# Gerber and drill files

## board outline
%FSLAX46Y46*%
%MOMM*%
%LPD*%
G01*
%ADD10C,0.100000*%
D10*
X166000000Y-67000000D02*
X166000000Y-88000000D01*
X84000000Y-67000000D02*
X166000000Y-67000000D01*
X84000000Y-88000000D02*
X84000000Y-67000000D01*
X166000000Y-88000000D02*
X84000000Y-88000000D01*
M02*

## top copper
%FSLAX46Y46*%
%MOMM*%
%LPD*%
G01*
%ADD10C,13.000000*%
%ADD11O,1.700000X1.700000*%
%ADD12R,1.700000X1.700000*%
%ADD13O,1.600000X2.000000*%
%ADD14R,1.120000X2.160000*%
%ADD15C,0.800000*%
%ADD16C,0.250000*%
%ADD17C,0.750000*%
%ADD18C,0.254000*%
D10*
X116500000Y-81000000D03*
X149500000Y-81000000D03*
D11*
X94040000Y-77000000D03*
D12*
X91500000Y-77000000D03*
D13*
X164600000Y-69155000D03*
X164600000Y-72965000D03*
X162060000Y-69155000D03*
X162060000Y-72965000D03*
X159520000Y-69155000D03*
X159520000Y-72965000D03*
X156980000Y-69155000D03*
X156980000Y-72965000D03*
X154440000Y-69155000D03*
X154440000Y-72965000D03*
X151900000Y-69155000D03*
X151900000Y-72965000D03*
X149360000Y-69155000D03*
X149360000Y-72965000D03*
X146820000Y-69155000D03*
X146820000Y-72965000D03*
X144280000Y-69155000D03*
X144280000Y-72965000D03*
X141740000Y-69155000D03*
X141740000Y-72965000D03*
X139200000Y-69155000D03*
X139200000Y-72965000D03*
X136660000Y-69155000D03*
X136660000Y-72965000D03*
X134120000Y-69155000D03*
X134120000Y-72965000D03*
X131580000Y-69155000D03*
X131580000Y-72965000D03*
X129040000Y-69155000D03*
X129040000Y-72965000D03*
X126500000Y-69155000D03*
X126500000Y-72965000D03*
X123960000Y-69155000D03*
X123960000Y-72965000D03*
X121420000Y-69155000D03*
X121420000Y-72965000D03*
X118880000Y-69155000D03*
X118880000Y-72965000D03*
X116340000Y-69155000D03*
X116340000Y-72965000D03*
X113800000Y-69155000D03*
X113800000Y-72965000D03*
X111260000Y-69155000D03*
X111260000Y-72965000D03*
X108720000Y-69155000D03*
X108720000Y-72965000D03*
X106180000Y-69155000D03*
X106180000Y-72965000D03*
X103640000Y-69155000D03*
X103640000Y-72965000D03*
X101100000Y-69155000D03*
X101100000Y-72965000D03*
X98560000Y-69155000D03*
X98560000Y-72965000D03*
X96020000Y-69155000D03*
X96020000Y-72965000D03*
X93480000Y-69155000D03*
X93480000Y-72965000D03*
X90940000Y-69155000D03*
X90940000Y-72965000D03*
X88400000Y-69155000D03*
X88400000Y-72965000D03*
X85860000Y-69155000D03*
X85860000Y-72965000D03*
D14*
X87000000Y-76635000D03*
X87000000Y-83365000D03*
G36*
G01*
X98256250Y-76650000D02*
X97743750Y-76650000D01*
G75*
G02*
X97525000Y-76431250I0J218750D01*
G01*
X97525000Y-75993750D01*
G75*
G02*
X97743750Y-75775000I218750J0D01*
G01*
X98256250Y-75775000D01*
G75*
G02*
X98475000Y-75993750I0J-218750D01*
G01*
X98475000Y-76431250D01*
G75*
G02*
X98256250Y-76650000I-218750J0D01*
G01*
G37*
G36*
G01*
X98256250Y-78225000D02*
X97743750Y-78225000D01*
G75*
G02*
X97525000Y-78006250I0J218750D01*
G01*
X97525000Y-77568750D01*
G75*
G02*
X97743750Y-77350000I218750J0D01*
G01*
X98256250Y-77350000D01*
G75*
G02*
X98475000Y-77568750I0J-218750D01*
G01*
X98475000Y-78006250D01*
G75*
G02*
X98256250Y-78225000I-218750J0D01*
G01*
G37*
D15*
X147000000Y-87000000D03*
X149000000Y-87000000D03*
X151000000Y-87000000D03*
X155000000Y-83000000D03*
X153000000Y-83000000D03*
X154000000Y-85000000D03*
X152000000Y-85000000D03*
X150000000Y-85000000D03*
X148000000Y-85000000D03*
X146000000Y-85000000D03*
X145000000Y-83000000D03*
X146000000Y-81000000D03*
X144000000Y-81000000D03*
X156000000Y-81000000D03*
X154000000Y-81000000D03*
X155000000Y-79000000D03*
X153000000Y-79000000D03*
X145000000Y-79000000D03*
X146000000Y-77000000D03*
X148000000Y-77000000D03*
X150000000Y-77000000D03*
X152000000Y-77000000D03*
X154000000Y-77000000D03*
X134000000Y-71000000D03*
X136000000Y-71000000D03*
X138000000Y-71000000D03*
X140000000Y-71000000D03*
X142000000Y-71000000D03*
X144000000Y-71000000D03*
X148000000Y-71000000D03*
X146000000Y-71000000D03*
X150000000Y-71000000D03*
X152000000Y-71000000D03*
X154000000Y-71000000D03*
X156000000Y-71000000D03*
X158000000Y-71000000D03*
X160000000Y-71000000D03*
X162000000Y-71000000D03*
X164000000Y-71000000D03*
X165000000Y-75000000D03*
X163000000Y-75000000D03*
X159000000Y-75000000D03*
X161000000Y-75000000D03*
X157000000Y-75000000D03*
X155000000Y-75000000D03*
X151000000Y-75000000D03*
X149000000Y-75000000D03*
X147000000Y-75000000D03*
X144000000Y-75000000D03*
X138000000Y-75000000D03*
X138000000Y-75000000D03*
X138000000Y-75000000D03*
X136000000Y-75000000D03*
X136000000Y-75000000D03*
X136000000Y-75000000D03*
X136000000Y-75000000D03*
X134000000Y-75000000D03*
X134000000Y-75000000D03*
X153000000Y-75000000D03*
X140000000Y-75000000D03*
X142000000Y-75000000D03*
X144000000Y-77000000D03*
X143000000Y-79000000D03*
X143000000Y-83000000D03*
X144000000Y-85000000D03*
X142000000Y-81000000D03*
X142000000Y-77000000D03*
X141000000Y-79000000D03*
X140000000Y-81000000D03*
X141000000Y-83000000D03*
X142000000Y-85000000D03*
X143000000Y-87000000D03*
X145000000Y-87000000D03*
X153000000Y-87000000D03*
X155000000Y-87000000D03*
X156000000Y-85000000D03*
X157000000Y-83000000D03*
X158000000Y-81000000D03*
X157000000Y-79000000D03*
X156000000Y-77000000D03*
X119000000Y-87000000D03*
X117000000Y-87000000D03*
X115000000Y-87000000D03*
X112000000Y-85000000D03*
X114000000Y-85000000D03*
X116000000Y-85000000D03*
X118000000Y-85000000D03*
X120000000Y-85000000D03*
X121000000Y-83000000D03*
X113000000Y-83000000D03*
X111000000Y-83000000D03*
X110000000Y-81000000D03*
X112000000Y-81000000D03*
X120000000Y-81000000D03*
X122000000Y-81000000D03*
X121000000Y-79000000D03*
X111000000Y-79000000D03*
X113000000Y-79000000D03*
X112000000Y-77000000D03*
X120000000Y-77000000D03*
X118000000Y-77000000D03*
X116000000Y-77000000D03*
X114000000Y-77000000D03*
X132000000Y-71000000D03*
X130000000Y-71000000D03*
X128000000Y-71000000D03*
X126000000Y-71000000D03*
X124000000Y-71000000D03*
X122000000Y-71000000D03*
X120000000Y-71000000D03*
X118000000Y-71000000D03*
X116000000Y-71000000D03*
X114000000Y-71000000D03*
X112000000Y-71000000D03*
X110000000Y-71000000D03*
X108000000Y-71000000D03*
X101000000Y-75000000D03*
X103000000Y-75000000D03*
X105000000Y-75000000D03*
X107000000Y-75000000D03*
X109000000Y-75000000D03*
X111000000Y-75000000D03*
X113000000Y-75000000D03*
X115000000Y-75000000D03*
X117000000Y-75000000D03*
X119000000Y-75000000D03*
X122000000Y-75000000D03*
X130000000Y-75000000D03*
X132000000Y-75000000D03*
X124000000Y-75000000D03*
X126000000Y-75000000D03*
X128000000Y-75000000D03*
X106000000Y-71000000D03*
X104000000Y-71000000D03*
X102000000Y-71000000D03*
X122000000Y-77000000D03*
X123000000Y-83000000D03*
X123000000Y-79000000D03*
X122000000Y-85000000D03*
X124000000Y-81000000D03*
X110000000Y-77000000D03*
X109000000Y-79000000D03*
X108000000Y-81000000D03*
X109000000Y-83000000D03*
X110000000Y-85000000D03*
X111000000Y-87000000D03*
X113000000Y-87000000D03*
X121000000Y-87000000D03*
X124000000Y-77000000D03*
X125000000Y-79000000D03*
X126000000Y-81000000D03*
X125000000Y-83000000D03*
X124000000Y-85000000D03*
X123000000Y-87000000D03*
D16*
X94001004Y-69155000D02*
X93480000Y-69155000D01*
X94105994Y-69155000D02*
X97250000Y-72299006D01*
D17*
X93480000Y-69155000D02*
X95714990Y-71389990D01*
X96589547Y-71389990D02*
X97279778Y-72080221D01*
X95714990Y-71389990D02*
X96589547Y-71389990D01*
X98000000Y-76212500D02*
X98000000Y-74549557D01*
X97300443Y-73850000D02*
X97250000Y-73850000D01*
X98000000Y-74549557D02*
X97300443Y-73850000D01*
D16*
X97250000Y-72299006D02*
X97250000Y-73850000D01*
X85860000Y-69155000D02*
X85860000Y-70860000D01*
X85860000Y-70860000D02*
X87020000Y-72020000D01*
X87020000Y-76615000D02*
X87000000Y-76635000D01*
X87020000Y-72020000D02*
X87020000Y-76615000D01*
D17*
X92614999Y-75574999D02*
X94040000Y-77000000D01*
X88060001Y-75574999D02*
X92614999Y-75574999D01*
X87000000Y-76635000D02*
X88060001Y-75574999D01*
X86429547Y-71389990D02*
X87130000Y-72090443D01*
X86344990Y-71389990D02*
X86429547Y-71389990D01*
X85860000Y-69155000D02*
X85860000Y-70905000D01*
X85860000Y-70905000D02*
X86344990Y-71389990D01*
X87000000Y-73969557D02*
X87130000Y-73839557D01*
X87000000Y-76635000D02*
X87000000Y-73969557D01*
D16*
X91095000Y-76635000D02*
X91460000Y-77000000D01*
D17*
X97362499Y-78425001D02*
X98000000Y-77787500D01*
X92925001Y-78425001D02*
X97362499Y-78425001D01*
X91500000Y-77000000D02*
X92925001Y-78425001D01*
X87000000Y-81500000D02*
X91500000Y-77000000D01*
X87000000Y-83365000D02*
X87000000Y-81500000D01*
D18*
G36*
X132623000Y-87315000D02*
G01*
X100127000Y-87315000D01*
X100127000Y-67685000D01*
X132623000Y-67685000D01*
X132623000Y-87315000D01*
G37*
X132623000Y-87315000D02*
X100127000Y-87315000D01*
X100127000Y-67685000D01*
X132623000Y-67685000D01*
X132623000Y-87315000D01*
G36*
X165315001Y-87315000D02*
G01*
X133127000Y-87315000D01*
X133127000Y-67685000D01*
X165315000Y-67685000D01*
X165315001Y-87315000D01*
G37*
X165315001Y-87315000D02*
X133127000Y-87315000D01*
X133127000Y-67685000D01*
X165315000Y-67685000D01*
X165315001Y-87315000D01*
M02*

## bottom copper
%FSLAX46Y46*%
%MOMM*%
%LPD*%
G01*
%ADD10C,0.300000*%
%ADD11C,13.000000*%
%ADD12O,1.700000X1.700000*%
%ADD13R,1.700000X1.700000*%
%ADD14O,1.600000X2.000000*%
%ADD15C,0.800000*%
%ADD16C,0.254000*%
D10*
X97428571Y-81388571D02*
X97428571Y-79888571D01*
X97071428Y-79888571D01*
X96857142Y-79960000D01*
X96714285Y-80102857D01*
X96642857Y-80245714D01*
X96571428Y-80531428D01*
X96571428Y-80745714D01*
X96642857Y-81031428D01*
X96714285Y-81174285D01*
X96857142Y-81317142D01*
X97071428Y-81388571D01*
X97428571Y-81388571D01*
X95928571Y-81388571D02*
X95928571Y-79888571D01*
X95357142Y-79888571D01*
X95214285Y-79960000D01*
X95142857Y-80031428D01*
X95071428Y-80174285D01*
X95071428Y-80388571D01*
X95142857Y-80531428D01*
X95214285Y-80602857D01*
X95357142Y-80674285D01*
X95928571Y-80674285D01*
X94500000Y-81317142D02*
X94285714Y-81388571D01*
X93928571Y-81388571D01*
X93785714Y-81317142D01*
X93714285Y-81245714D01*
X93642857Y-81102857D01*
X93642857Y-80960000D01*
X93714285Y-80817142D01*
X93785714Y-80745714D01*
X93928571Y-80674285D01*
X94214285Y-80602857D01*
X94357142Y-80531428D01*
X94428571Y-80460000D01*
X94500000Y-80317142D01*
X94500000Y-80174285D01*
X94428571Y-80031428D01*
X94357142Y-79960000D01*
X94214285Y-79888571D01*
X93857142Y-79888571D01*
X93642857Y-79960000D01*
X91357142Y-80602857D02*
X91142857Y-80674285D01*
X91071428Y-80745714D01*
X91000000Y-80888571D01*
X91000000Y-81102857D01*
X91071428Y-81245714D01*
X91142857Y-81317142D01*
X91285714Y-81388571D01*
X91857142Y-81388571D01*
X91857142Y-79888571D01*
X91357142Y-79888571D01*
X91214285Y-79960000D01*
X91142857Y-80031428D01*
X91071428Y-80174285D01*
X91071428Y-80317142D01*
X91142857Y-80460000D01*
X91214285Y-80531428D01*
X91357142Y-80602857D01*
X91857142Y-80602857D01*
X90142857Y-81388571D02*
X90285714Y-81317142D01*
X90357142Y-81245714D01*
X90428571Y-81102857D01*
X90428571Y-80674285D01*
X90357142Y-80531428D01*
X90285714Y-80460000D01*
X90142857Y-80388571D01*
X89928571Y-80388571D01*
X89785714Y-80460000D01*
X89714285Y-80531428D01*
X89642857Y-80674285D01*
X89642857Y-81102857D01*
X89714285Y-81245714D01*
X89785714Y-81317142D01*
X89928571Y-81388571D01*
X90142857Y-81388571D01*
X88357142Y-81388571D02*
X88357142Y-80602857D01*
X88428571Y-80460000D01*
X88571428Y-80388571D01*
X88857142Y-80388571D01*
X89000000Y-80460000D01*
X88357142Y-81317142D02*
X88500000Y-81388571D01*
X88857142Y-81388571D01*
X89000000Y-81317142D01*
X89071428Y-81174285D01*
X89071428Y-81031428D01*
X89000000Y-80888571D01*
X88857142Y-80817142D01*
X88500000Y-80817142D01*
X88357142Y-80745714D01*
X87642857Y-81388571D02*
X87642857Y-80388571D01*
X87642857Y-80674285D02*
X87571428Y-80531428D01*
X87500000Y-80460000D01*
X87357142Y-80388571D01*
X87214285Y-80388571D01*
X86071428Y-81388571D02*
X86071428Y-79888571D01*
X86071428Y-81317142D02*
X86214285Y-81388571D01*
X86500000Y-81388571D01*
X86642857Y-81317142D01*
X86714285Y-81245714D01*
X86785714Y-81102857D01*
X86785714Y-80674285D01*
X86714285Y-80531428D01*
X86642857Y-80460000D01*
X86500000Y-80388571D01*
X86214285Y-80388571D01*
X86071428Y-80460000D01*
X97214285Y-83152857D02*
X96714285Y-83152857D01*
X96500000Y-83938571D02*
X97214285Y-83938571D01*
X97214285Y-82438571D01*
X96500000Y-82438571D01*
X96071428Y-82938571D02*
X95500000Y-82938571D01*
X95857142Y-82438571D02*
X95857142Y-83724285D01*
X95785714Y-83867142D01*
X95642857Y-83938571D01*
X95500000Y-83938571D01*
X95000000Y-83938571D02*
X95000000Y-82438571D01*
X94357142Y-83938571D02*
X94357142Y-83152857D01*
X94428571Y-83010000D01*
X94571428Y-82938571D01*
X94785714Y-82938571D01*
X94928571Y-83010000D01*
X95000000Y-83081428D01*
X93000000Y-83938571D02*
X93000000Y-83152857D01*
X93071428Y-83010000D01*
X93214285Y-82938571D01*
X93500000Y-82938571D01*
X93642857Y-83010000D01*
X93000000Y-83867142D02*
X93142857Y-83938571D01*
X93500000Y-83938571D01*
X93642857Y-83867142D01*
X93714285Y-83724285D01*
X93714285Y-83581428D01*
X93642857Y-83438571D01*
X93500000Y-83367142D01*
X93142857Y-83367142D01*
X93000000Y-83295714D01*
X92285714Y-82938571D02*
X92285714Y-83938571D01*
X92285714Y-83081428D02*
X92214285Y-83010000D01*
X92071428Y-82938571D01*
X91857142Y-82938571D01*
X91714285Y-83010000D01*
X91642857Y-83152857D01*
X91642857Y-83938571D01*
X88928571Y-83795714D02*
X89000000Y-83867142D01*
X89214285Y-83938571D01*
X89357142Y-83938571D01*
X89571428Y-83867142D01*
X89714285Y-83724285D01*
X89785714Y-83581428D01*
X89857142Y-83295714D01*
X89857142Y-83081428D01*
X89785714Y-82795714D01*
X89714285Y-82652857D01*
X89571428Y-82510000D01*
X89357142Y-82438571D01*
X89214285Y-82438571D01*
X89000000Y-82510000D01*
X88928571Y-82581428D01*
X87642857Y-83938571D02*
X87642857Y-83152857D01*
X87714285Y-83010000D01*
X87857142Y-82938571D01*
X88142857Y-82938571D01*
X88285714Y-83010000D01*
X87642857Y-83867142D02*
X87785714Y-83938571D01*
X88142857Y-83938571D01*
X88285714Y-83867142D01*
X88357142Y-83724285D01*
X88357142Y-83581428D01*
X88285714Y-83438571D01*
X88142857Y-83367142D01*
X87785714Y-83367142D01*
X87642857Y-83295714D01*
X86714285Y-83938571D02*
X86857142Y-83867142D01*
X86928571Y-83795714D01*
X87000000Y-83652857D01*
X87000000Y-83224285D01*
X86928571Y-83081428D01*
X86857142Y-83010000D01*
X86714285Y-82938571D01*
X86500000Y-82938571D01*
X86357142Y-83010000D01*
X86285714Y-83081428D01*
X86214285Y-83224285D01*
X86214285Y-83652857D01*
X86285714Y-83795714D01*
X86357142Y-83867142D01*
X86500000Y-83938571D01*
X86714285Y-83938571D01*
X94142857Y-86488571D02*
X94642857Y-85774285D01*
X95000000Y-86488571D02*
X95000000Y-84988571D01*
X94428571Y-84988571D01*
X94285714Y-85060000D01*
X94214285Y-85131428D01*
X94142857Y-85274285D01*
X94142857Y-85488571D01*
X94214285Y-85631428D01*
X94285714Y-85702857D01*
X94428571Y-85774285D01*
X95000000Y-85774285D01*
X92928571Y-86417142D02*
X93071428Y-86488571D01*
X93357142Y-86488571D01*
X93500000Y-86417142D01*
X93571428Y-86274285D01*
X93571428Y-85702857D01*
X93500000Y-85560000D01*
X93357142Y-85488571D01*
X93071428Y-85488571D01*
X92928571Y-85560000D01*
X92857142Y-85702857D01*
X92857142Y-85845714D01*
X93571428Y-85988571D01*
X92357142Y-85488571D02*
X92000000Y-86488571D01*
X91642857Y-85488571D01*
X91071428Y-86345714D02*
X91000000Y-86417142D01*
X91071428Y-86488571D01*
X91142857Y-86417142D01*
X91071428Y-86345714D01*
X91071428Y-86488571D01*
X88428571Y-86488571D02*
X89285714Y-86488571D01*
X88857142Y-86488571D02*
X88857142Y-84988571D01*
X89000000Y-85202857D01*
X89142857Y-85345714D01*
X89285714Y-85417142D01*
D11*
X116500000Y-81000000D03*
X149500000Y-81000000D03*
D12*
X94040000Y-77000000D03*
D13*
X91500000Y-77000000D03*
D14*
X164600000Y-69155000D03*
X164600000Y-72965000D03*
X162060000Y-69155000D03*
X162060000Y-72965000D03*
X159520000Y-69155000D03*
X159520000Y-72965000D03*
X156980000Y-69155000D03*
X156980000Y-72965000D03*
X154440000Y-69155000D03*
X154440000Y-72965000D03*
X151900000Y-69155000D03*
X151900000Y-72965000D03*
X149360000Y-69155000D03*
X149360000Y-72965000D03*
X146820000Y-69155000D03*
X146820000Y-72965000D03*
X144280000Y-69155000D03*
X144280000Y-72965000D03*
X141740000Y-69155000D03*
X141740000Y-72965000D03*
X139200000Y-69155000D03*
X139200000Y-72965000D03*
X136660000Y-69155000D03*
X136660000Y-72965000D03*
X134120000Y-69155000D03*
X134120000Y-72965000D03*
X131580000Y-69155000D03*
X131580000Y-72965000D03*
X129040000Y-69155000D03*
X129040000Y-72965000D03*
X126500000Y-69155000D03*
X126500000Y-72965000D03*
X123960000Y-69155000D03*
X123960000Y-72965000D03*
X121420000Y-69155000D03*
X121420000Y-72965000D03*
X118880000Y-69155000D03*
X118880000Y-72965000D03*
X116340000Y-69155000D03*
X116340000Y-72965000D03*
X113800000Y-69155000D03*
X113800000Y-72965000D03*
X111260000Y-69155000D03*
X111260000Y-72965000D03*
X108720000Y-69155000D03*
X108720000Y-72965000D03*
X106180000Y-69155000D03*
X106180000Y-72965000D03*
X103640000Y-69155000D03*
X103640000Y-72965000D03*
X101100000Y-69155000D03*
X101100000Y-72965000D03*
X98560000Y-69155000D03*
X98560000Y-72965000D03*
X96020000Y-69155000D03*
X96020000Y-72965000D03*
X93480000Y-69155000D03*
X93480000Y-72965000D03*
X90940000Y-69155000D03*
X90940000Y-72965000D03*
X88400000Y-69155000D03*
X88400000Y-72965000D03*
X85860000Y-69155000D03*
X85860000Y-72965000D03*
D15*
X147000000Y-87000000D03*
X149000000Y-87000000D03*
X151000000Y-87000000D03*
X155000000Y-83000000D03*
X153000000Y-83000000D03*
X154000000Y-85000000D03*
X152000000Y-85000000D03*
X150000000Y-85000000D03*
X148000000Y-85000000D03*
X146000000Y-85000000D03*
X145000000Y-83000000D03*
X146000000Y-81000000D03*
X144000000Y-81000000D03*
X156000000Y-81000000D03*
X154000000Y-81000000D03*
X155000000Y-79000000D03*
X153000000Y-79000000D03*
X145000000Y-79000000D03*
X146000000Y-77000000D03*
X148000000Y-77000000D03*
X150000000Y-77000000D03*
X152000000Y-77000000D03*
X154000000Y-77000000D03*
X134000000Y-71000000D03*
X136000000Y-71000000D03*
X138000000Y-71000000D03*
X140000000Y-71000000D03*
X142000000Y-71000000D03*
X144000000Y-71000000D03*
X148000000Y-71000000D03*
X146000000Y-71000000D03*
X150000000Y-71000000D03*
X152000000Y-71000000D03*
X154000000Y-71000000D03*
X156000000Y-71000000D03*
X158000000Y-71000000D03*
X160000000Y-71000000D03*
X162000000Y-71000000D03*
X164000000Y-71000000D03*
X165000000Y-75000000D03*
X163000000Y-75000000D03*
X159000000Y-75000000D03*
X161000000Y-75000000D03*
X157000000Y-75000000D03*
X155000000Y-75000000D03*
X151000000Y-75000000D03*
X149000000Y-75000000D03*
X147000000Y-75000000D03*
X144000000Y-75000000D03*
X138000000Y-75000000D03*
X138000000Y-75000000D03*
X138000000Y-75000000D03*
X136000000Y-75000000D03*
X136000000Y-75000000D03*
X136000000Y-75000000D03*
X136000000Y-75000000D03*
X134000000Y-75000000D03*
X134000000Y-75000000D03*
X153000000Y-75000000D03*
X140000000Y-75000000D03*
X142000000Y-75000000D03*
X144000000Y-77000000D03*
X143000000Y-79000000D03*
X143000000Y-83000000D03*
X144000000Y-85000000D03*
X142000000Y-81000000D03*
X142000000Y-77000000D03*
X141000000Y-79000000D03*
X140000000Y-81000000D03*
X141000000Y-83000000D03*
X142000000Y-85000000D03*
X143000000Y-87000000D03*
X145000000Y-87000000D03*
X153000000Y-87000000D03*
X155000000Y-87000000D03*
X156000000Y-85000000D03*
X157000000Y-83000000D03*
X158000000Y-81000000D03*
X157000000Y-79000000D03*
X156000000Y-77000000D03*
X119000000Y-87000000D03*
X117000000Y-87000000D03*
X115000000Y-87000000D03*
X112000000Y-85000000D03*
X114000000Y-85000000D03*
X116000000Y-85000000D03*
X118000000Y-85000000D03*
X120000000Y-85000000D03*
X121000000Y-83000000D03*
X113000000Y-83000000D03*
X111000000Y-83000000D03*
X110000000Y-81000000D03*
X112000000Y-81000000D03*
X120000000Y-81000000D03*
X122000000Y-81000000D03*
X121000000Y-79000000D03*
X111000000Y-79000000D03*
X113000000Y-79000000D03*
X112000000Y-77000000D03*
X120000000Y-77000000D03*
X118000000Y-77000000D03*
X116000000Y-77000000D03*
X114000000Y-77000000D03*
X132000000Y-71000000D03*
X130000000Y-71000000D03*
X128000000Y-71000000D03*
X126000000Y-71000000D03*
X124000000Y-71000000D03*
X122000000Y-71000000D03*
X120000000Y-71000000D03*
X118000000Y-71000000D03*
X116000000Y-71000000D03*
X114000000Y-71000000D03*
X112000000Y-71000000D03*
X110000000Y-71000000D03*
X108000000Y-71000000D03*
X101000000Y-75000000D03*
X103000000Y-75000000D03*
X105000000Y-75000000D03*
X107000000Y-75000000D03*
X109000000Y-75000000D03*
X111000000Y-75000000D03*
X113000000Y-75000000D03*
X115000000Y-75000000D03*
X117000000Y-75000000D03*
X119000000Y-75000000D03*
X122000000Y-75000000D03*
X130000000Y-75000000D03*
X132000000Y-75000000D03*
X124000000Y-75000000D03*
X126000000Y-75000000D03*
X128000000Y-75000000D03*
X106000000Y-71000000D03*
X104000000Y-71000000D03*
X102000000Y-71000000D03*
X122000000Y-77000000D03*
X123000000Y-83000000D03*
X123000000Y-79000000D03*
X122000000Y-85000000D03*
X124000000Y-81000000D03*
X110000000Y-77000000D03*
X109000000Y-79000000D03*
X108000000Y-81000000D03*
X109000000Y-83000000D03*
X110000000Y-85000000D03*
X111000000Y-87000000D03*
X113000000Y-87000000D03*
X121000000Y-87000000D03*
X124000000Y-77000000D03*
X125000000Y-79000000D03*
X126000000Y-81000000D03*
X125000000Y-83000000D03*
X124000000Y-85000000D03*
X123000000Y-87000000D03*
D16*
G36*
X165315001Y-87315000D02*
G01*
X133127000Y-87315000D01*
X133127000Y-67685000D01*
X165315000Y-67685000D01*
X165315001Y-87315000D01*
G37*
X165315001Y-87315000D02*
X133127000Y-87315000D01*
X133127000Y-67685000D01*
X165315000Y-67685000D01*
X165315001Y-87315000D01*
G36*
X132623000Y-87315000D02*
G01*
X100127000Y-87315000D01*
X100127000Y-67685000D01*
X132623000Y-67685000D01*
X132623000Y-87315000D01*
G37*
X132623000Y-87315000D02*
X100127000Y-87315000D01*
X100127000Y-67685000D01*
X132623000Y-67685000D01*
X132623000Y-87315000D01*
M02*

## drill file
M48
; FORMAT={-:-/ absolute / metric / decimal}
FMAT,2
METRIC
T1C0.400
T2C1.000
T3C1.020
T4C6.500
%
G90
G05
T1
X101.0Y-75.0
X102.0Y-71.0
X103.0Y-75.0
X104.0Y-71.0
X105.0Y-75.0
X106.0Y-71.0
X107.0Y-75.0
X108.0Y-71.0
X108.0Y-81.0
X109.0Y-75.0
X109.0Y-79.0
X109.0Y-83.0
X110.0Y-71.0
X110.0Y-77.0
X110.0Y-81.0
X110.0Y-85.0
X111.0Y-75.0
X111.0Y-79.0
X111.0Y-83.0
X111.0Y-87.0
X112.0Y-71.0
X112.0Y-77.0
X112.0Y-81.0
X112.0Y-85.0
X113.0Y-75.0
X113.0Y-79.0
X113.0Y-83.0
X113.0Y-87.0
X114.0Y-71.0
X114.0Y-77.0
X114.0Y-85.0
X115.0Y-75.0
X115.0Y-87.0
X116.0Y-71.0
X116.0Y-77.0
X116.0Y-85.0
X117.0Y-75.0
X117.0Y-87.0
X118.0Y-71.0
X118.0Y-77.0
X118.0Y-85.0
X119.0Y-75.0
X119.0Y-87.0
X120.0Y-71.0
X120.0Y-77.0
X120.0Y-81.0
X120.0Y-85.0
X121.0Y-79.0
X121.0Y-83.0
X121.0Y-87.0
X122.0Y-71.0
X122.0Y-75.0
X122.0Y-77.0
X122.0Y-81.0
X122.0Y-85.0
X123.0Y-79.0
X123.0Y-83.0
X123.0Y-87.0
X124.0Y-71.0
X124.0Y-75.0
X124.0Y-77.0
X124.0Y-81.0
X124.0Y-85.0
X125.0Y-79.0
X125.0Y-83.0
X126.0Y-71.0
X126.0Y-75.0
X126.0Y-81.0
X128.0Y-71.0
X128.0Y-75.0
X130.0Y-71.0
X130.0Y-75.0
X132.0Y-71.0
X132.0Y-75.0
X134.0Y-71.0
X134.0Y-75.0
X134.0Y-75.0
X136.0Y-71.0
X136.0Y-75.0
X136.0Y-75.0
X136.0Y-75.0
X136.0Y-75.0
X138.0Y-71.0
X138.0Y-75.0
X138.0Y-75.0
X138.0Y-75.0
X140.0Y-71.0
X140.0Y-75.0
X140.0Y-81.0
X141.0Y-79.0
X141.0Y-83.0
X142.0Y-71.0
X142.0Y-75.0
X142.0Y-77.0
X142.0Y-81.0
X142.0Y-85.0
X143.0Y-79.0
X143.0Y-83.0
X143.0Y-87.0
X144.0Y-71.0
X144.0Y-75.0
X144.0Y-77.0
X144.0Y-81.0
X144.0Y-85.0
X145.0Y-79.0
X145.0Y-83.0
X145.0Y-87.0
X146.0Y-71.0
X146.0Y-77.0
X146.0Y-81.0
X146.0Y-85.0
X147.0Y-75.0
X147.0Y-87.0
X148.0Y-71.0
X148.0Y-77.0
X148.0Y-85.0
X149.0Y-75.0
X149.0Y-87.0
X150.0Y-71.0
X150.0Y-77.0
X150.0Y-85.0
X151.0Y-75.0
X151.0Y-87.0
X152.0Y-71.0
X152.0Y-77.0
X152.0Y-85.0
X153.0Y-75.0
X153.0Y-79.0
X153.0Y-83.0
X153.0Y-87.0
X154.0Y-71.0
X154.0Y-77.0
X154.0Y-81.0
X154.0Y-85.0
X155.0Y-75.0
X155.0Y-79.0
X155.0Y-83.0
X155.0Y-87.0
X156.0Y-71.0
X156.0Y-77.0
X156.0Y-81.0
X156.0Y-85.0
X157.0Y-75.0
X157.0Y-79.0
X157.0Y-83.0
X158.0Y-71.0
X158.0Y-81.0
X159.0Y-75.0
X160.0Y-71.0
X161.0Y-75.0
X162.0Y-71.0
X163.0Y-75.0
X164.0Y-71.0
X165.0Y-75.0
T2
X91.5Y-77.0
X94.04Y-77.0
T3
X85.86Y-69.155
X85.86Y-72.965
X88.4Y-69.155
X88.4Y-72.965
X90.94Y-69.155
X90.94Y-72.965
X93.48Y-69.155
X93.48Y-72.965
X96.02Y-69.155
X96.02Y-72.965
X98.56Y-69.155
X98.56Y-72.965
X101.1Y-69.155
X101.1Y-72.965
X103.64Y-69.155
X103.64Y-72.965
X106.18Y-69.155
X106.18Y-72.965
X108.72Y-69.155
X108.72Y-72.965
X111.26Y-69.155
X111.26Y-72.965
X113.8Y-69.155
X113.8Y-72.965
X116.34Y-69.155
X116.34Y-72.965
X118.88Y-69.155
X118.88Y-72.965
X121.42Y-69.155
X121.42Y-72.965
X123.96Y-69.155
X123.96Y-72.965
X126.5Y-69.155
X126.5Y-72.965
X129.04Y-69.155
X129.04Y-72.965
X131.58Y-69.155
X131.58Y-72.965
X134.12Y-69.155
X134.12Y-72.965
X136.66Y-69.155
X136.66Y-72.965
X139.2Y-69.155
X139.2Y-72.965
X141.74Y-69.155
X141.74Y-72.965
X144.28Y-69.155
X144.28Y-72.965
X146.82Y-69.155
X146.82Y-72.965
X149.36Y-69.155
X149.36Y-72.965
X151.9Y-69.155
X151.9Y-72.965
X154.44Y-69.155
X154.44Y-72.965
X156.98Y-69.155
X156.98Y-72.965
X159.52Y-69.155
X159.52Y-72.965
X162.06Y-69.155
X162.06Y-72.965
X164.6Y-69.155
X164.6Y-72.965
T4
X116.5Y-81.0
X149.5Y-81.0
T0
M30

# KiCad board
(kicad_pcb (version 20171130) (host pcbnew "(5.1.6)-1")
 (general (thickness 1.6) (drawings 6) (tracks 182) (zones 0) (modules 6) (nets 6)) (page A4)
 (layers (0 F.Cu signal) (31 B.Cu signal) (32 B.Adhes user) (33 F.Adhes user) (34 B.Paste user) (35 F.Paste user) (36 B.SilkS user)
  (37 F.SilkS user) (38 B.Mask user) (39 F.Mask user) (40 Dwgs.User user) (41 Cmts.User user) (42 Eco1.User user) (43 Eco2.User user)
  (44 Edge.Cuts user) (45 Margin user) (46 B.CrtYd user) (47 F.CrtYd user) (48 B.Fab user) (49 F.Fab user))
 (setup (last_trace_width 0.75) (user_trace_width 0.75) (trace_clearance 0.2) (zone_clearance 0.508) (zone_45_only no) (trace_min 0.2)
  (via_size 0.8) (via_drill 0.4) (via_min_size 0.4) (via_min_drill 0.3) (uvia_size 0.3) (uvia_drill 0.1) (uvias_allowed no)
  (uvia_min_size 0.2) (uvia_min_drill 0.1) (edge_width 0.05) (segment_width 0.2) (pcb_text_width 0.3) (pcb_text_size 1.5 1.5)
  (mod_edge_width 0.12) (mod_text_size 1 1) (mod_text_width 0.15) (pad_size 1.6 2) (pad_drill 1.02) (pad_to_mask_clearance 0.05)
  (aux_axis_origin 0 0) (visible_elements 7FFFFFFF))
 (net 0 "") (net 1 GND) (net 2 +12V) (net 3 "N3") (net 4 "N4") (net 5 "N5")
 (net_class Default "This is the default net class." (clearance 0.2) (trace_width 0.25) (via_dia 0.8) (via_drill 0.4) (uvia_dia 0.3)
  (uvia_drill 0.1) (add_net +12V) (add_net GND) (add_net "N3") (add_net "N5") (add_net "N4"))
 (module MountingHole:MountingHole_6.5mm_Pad (layer F.Cu) (at 116.5 81)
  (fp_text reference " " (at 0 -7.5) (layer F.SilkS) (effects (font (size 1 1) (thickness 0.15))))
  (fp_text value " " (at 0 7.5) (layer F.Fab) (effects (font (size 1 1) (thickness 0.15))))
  (pad 1 thru_hole circle (at 0 0) (size 13 13) (drill 6.5) (layers *.Cu *.Mask) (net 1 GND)))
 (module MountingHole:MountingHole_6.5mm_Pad (layer F.Cu) (at 149.5 81)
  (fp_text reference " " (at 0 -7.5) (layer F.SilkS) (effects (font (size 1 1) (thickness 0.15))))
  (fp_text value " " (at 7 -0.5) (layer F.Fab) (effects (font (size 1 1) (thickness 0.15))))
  (pad 1 thru_hole circle (at 0 0) (size 13 13) (drill 6.5) (layers *.Cu *.Mask) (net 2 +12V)))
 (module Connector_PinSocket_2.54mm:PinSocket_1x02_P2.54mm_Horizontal (layer F.Cu) (at 91.5 77 90)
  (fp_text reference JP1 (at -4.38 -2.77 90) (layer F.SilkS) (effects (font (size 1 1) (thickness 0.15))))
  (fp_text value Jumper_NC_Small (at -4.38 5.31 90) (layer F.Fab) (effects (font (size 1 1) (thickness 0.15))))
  (pad 2 thru_hole oval (at 0 2.54 90) (size 1.7 1.7) (drill 1) (layers *.Cu *.Mask) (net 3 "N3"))
  (pad 1 thru_hole rect (at 0 0 90) (size 1.7 1.7) (drill 1) (layers *.Cu *.Mask) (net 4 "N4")))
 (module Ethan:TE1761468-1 (layer B.Cu) (at 125.23 71.06)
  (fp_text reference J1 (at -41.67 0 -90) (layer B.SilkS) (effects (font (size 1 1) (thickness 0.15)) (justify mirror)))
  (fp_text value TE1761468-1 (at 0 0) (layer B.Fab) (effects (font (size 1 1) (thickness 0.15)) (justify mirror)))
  (pad 32 thru_hole oval (at 39.37 -1.905) (size 1.6 2) (drill 1.02) (layers *.Cu *.Mask) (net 2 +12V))
  (pad 33 thru_hole oval (at 39.37 1.905) (size 1.6 2) (drill 1.02) (layers *.Cu *.Mask) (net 2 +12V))
  (pad 31 thru_hole oval (at 36.83 -1.905) (size 1.6 2) (drill 1.02) (layers *.Cu *.Mask) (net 2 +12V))
  (pad 34 thru_hole oval (at 36.83 1.905) (size 1.6 2) (drill 1.02) (layers *.Cu *.Mask) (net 2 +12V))
  (pad 30 thru_hole oval (at 34.29 -1.905) (size 1.6 2) (drill 1.02) (layers *.Cu *.Mask) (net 2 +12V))
  (pad 35 thru_hole oval (at 34.29 1.905) (size 1.6 2) (drill 1.02) (layers *.Cu *.Mask) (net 2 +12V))
  (pad 29 thru_hole oval (at 31.75 -1.905) (size 1.6 2) (drill 1.02) (layers *.Cu *.Mask) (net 2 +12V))
  (pad 36 thru_hole oval (at 31.75 1.905) (size 1.6 2) (drill 1.02) (layers *.Cu *.Mask) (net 2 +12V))
  (pad 28 thru_hole oval (at 29.21 -1.905) (size 1.6 2) (drill 1.02) (layers *.Cu *.Mask) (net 2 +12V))
  (pad 37 thru_hole oval (at 29.21 1.905) (size 1.6 2) (drill 1.02) (layers *.Cu *.Mask) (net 2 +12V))
  (pad 27 thru_hole oval (at 26.67 -1.905) (size 1.6 2) (drill 1.02) (layers *.Cu *.Mask) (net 2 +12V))
  (pad 38 thru_hole oval (at 26.67 1.905) (size 1.6 2) (drill 1.02) (layers *.Cu *.Mask) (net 2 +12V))
  (pad 26 thru_hole oval (at 24.13 -1.905) (size 1.6 2) (drill 1.02) (layers *.Cu *.Mask) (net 2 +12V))
  (pad 39 thru_hole oval (at 24.13 1.905) (size 1.6 2) (drill 1.02) (layers *.Cu *.Mask) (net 2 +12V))
  (pad 25 thru_hole oval (at 21.59 -1.905) (size 1.6 2) (drill 1.02) (layers *.Cu *.Mask) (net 2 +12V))
  (pad 40 thru_hole oval (at 21.59 1.905) (size 1.6 2) (drill 1.02) (layers *.Cu *.Mask) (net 2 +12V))
  (pad 24 thru_hole oval (at 19.05 -1.905) (size 1.6 2) (drill 1.02) (layers *.Cu *.Mask) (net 2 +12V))
  (pad 41 thru_hole oval (at 19.05 1.905) (size 1.6 2) (drill 1.02) (layers *.Cu *.Mask) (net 2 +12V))
  (pad 23 thru_hole oval (at 16.51 -1.905) (size 1.6 2) (drill 1.02) (layers *.Cu *.Mask) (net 2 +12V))
  (pad 42 thru_hole oval (at 16.51 1.905) (size 1.6 2) (drill 1.02) (layers *.Cu *.Mask) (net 2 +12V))
  (pad 22 thru_hole oval (at 13.97 -1.905) (size 1.6 2) (drill 1.02) (layers *.Cu *.Mask) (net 2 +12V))
  (pad 43 thru_hole oval (at 13.97 1.905) (size 1.6 2) (drill 1.02) (layers *.Cu *.Mask) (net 2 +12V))
  (pad 21 thru_hole oval (at 11.43 -1.905) (size 1.6 2) (drill 1.02) (layers *.Cu *.Mask) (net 2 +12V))
  (pad 44 thru_hole oval (at 11.43 1.905) (size 1.6 2) (drill 1.02) (layers *.Cu *.Mask) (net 2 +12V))
  (pad 20 thru_hole oval (at 8.89 -1.905) (size 1.6 2) (drill 1.02) (layers *.Cu *.Mask) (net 2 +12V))
  (pad 45 thru_hole oval (at 8.89 1.905) (size 1.6 2) (drill 1.02) (layers *.Cu *.Mask) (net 2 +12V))
  (pad 19 thru_hole oval (at 6.35 -1.905) (size 1.6 2) (drill 1.02) (layers *.Cu *.Mask) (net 1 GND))
  (pad 46 thru_hole oval (at 6.35 1.905) (size 1.6 2) (drill 1.02) (layers *.Cu *.Mask) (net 1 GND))
  (pad 18 thru_hole oval (at 3.81 -1.905) (size 1.6 2) (drill 1.02) (layers *.Cu *.Mask) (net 1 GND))
  (pad 47 thru_hole oval (at 3.81 1.905) (size 1.6 2) (drill 1.02) (layers *.Cu *.Mask) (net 1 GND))
  (pad 17 thru_hole oval (at 1.27 -1.905) (size 1.6 2) (drill 1.02) (layers *.Cu *.Mask) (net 1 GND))
  (pad 48 thru_hole oval (at 1.27 1.905) (size 1.6 2) (drill 1.02) (layers *.Cu *.Mask) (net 1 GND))
  (pad 16 thru_hole oval (at -1.27 -1.905) (size 1.6 2) (drill 1.02) (layers *.Cu *.Mask) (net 1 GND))
  (pad 49 thru_hole oval (at -1.27 1.905) (size 1.6 2) (drill 1.02) (layers *.Cu *.Mask) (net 1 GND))
  (pad 15 thru_hole oval (at -3.81 -1.905) (size 1.6 2) (drill 1.02) (layers *.Cu *.Mask) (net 1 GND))
  (pad 50 thru_hole oval (at -3.81 1.905) (size 1.6 2) (drill 1.02) (layers *.Cu *.Mask) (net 1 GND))
  (pad 14 thru_hole oval (at -6.35 -1.905) (size 1.6 2) (drill 1.02) (layers *.Cu *.Mask) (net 1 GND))
  (pad 51 thru_hole oval (at -6.35 1.905) (size 1.6 2) (drill 1.02) (layers *.Cu *.Mask) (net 1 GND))
  (pad 13 thru_hole oval (at -8.89 -1.905) (size 1.6 2) (drill 1.02) (layers *.Cu *.Mask) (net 1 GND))
  (pad 52 thru_hole oval (at -8.89 1.905) (size 1.6 2) (drill 1.02) (layers *.Cu *.Mask) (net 1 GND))
  (pad 12 thru_hole oval (at -11.43 -1.905) (size 1.6 2) (drill 1.02) (layers *.Cu *.Mask) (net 1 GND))
  (pad 53 thru_hole oval (at -11.43 1.905) (size 1.6 2) (drill 1.02) (layers *.Cu *.Mask) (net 1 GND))
  (pad 11 thru_hole oval (at -13.97 -1.905) (size 1.6 2) (drill 1.02) (layers *.Cu *.Mask) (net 1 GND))
  (pad 54 thru_hole oval (at -13.97 1.905) (size 1.6 2) (drill 1.02) (layers *.Cu *.Mask) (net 1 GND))
  (pad 10 thru_hole oval (at -16.51 -1.905) (size 1.6 2) (drill 1.02) (layers *.Cu *.Mask) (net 1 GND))
  (pad 55 thru_hole oval (at -16.51 1.905) (size 1.6 2) (drill 1.02) (layers *.Cu *.Mask) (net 1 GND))
  (pad 9 thru_hole oval (at -19.05 -1.905) (size 1.6 2) (drill 1.02) (layers *.Cu *.Mask) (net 1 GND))
  (pad 56 thru_hole oval (at -19.05 1.905) (size 1.6 2) (drill 1.02) (layers *.Cu *.Mask) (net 1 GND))
  (pad 8 thru_hole oval (at -21.59 -1.905) (size 1.6 2) (drill 1.02) (layers *.Cu *.Mask) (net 1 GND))
  (pad 57 thru_hole oval (at -21.59 1.905) (size 1.6 2) (drill 1.02) (layers *.Cu *.Mask) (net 1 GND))
  (pad 7 thru_hole oval (at -24.13 -1.905) (size 1.6 2) (drill 1.02) (layers *.Cu *.Mask) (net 1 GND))
  (pad 58 thru_hole oval (at -24.13 1.905) (size 1.6 2) (drill 1.02) (layers *.Cu *.Mask) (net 1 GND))
  (pad 6 thru_hole oval (at -26.67 -1.905) (size 1.6 2) (drill 1.02) (layers *.Cu *.Mask))
  (pad 59 thru_hole oval (at -26.67 1.905) (size 1.6 2) (drill 1.02) (layers *.Cu *.Mask))
  (pad 5 thru_hole oval (at -29.21 -1.905) (size 1.6 2) (drill 1.02) (layers *.Cu *.Mask))
  (pad 60 thru_hole oval (at -29.21 1.905) (size 1.6 2) (drill 1.02) (layers *.Cu *.Mask))
  (pad 4 thru_hole oval (at -31.75 -1.905) (size 1.6 2) (drill 1.02) (layers *.Cu *.Mask) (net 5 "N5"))
  (pad 61 thru_hole oval (at -31.75 1.905) (size 1.6 2) (drill 1.02) (layers *.Cu *.Mask))
  (pad 3 thru_hole oval (at -34.29 -1.905) (size 1.6 2) (drill 1.02) (layers *.Cu *.Mask))
  (pad 62 thru_hole oval (at -34.29 1.905) (size 1.6 2) (drill 1.02) (layers *.Cu *.Mask))
  (pad 2 thru_hole oval (at -36.83 -1.905) (size 1.6 2) (drill 1.02) (layers *.Cu *.Mask))
  (pad 63 thru_hole oval (at -36.83 1.905) (size 1.6 2) (drill 1.02) (layers *.Cu *.Mask))
  (pad 1 thru_hole oval (at -39.37 -1.905) (size 1.6 2) (drill 1.02) (layers *.Cu *.Mask) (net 3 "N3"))
  (pad 64 thru_hole oval (at -39.37 1.905) (size 1.6 2) (drill 1.02) (layers *.Cu *.Mask)))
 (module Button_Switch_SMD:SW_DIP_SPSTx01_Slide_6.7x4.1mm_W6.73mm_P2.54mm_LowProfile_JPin (layer F.Cu) (at 87 80 90)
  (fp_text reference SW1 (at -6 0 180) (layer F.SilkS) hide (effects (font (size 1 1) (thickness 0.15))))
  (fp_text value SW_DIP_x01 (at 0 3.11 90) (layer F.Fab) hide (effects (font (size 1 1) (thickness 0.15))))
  (pad 2 smd rect (at 3.365 0 90) (size 2.16 1.12) (layers F.Cu F.Paste F.Mask) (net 3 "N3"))
  (pad 1 smd rect (at -3.365 0 90) (size 2.16 1.12) (layers F.Cu F.Paste F.Mask) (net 4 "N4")))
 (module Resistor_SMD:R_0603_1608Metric (layer F.Cu) (at 98 77 90)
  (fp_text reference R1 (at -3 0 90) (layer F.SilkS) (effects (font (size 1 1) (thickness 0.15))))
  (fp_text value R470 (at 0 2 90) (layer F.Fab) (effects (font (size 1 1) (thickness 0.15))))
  (pad 2 smd roundrect (at 0.7875 0 90) (size 0.875 0.95) (layers F.Cu F.Paste F.Mask) (roundrect_rratio 0.25) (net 5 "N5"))
  (pad 1 smd roundrect (at -0.7875 0 90) (size 0.875 0.95) (layers F.Cu F.Paste F.Mask) (roundrect_rratio 0.25) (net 4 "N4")))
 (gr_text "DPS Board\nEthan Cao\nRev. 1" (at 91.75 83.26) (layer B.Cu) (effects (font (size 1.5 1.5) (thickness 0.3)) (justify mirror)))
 (gr_line (start 166 67) (end 166 88) (layer Edge.Cuts) (width 0.1))
 (gr_line (start 84 67) (end 166 67) (layer Edge.Cuts) (width 0.1))
 (gr_line (start 84 88) (end 84 67) (layer Edge.Cuts) (width 0.1))
 (gr_line (start 166 88) (end 84 88) (layer Edge.Cuts) (width 0.1))
 (via (at 147 87) (size 0.8) (drill 0.4) (layers F.Cu B.Cu) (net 2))
 (via (at 149 87) (size 0.8) (drill 0.4) (layers F.Cu B.Cu) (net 2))
 (via (at 151 87) (size 0.8) (drill 0.4) (layers F.Cu B.Cu) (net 2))
 (via (at 155 83) (size 0.8) (drill 0.4) (layers F.Cu B.Cu) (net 2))
 (via (at 153 83) (size 0.8) (drill 0.4) (layers F.Cu B.Cu) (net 2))
 (via (at 154 85) (size 0.8) (drill 0.4) (layers F.Cu B.Cu) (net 2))
 (via (at 152 85) (size 0.8) (drill 0.4) (layers F.Cu B.Cu) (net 2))
 (via (at 150 85) (size 0.8) (drill 0.4) (layers F.Cu B.Cu) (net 2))
 (via (at 148 85) (size 0.8) (drill 0.4) (layers F.Cu B.Cu) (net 2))
 (via (at 146 85) (size 0.8) (drill 0.4) (layers F.Cu B.Cu) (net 2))
 (via (at 145 83) (size 0.8) (drill 0.4) (layers F.Cu B.Cu) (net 2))
 (via (at 146 81) (size 0.8) (drill 0.4) (layers F.Cu B.Cu) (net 2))
 (via (at 144 81) (size 0.8) (drill 0.4) (layers F.Cu B.Cu) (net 2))
 (via (at 156 81) (size 0.8) (drill 0.4) (layers F.Cu B.Cu) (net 2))
 (via (at 154 81) (size 0.8) (drill 0.4) (layers F.Cu B.Cu) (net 2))
 (via (at 155 79) (size 0.8) (drill 0.4) (layers F.Cu B.Cu) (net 2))
 (via (at 153 79) (size 0.8) (drill 0.4) (layers F.Cu B.Cu) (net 2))
 (via (at 145 79) (size 0.8) (drill 0.4) (layers F.Cu B.Cu) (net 2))
 (via (at 146 77) (size 0.8) (drill 0.4) (layers F.Cu B.Cu) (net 2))
 (via (at 148 77) (size 0.8) (drill 0.4) (layers F.Cu B.Cu) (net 2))
 (via (at 150 77) (size 0.8) (drill 0.4) (layers F.Cu B.Cu) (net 2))
 (via (at 152 77) (size 0.8) (drill 0.4) (layers F.Cu B.Cu) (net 2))
 (via (at 154 77) (size 0.8) (drill 0.4) (layers F.Cu B.Cu) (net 2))
 (via (at 134 71) (size 0.8) (drill 0.4) (layers F.Cu B.Cu) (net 2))
 (via (at 136 71) (size 0.8) (drill 0.4) (layers F.Cu B.Cu) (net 2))
 (via (at 138 71) (size 0.8) (drill 0.4) (layers F.Cu B.Cu) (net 2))
 (via (at 140 71) (size 0.8) (drill 0.4) (layers F.Cu B.Cu) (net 2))
 (via (at 142 71) (size 0.8) (drill 0.4) (layers F.Cu B.Cu) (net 2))
 (via (at 144 71) (size 0.8) (drill 0.4) (layers F.Cu B.Cu) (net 2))
 (via (at 148 71) (size 0.8) (drill 0.4) (layers F.Cu B.Cu) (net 2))
 (via (at 146 71) (size 0.8) (drill 0.4) (layers F.Cu B.Cu) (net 2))
 (via (at 150 71) (size 0.8) (drill 0.4) (layers F.Cu B.Cu) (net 2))
 (via (at 152 71) (size 0.8) (drill 0.4) (layers F.Cu B.Cu) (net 2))
 (via (at 154 71) (size 0.8) (drill 0.4) (layers F.Cu B.Cu) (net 2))
 (via (at 156 71) (size 0.8) (drill 0.4) (layers F.Cu B.Cu) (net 2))
 (via (at 158 71) (size 0.8) (drill 0.4) (layers F.Cu B.Cu) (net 2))
 (via (at 160 71) (size 0.8) (drill 0.4) (layers F.Cu B.Cu) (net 2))
 (via (at 162 71) (size 0.8) (drill 0.4) (layers F.Cu B.Cu) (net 2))
 (via (at 164 71) (size 0.8) (drill 0.4) (layers F.Cu B.Cu) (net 2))
 (via (at 165 75) (size 0.8) (drill 0.4) (layers F.Cu B.Cu) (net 2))
 (via (at 163 75) (size 0.8) (drill 0.4) (layers F.Cu B.Cu) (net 2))
 (via (at 159 75) (size 0.8) (drill 0.4) (layers F.Cu B.Cu) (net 2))
 (via (at 161 75) (size 0.8) (drill 0.4) (layers F.Cu B.Cu) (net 2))
 (via (at 157 75) (size 0.8) (drill 0.4) (layers F.Cu B.Cu) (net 2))
 (via (at 155 75) (size 0.8) (drill 0.4) (layers F.Cu B.Cu) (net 2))
 (via (at 151 75) (size 0.8) (drill 0.4) (layers F.Cu B.Cu) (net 2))
 (via (at 149 75) (size 0.8) (drill 0.4) (layers F.Cu B.Cu) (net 2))
 (via (at 147 75) (size 0.8) (drill 0.4) (layers F.Cu B.Cu) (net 2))
 (via (at 144 75) (size 0.8) (drill 0.4) (layers F.Cu B.Cu) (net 2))
 (via (at 138 75) (size 0.8) (drill 0.4) (layers F.Cu B.Cu) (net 2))
 (via (at 138 75) (size 0.8) (drill 0.4) (layers F.Cu B.Cu) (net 2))
 (via (at 138 75) (size 0.8) (drill 0.4) (layers F.Cu B.Cu) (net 2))
 (via (at 136 75) (size 0.8) (drill 0.4) (layers F.Cu B.Cu) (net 2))
 (via (at 136 75) (size 0.8) (drill 0.4) (layers F.Cu B.Cu) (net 2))
 (via (at 136 75) (size 0.8) (drill 0.4) (layers F.Cu B.Cu) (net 2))
 (via (at 136 75) (size 0.8) (drill 0.4) (layers F.Cu B.Cu) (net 2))
 (via (at 134 75) (size 0.8) (drill 0.4) (layers F.Cu B.Cu) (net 2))
 (via (at 134 75) (size 0.8) (drill 0.4) (layers F.Cu B.Cu) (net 2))
 (via (at 153 75) (size 0.8) (drill 0.4) (layers F.Cu B.Cu) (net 2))
 (via (at 140 75) (size 0.8) (drill 0.4) (layers F.Cu B.Cu) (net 2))
 (via (at 142 75) (size 0.8) (drill 0.4) (layers F.Cu B.Cu) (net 2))
 (via (at 144 77) (size 0.8) (drill 0.4) (layers F.Cu B.Cu) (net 2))
 (via (at 143 79) (size 0.8) (drill 0.4) (layers F.Cu B.Cu) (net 2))
 (via (at 143 83) (size 0.8) (drill 0.4) (layers F.Cu B.Cu) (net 2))
 (via (at 144 85) (size 0.8) (drill 0.4) (layers F.Cu B.Cu) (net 2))
 (via (at 142 81) (size 0.8) (drill 0.4) (layers F.Cu B.Cu) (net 2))
 (via (at 142 77) (size 0.8) (drill 0.4) (layers F.Cu B.Cu) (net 2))
 (via (at 141 79) (size 0.8) (drill 0.4) (layers F.Cu B.Cu) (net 2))
 (via (at 140 81) (size 0.8) (drill 0.4) (layers F.Cu B.Cu) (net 2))
 (via (at 141 83) (size 0.8) (drill 0.4) (layers F.Cu B.Cu) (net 2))
 (via (at 142 85) (size 0.8) (drill 0.4) (layers F.Cu B.Cu) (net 2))
 (via (at 143 87) (size 0.8) (drill 0.4) (layers F.Cu B.Cu) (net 2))
 (via (at 145 87) (size 0.8) (drill 0.4) (layers F.Cu B.Cu) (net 2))
 (via (at 153 87) (size 0.8) (drill 0.4) (layers F.Cu B.Cu) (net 2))
 (via (at 155 87) (size 0.8) (drill 0.4) (layers F.Cu B.Cu) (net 2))
 (via (at 156 85) (size 0.8) (drill 0.4) (layers F.Cu B.Cu) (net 2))
 (via (at 157 83) (size 0.8) (drill 0.4) (layers F.Cu B.Cu) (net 2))
 (via (at 158 81) (size 0.8) (drill 0.4) (layers F.Cu B.Cu) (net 2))
 (via (at 157 79) (size 0.8) (drill 0.4) (layers F.Cu B.Cu) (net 2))
 (via (at 156 77) (size 0.8) (drill 0.4) (layers F.Cu B.Cu) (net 2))
 (via (at 119 87) (size 0.8) (drill 0.4) (layers F.Cu B.Cu) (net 1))
 (via (at 117 87) (size 0.8) (drill 0.4) (layers F.Cu B.Cu) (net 1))
 (via (at 115 87) (size 0.8) (drill 0.4) (layers F.Cu B.Cu) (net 1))
 (via (at 112 85) (size 0.8) (drill 0.4) (layers F.Cu B.Cu) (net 1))
 (via (at 114 85) (size 0.8) (drill 0.4) (layers F.Cu B.Cu) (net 1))
 (via (at 116 85) (size 0.8) (drill 0.4) (layers F.Cu B.Cu) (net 1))
 (via (at 118 85) (size 0.8) (drill 0.4) (layers F.Cu B.Cu) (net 1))
 (via (at 120 85) (size 0.8) (drill 0.4) (layers F.Cu B.Cu) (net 1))
 (via (at 121 83) (size 0.8) (drill 0.4) (layers F.Cu B.Cu) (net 1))
 (via (at 113 83) (size 0.8) (drill 0.4) (layers F.Cu B.Cu) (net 1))
 (via (at 111 83) (size 0.8) (drill 0.4) (layers F.Cu B.Cu) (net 1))
 (via (at 110 81) (size 0.8) (drill 0.4) (layers F.Cu B.Cu) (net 1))
 (via (at 112 81) (size 0.8) (drill 0.4) (layers F.Cu B.Cu) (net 1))
 (via (at 120 81) (size 0.8) (drill 0.4) (layers F.Cu B.Cu) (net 1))
 (via (at 122 81) (size 0.8) (drill 0.4) (layers F.Cu B.Cu) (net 1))
 (via (at 121 79) (size 0.8) (drill 0.4) (layers F.Cu B.Cu) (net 1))
 (via (at 111 79) (size 0.8) (drill 0.4) (layers F.Cu B.Cu) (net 1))
 (via (at 113 79) (size 0.8) (drill 0.4) (layers F.Cu B.Cu) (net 1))
 (via (at 112 77) (size 0.8) (drill 0.4) (layers F.Cu B.Cu) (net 1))
 (via (at 120 77) (size 0.8) (drill 0.4) (layers F.Cu B.Cu) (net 1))
 (via (at 118 77) (size 0.8) (drill 0.4) (layers F.Cu B.Cu) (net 1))
 (via (at 116 77) (size 0.8) (drill 0.4) (layers F.Cu B.Cu) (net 1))
 (via (at 114 77) (size 0.8) (drill 0.4) (layers F.Cu B.Cu) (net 1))
 (via (at 132 71) (size 0.8) (drill 0.4) (layers F.Cu B.Cu) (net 1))
 (via (at 130 71) (size 0.8) (drill 0.4) (layers F.Cu B.Cu) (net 1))
 (via (at 128 71) (size 0.8) (drill 0.4) (layers F.Cu B.Cu) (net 1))
 (via (at 126 71) (size 0.8) (drill 0.4) (layers F.Cu B.Cu) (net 1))
 (via (at 124 71) (size 0.8) (drill 0.4) (layers F.Cu B.Cu) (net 1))
 (via (at 122 71) (size 0.8) (drill 0.4) (layers F.Cu B.Cu) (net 1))
 (via (at 120 71) (size 0.8) (drill 0.4) (layers F.Cu B.Cu) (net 1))
 (via (at 118 71) (size 0.8) (drill 0.4) (layers F.Cu B.Cu) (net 1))
 (via (at 116 71) (size 0.8) (drill 0.4) (layers F.Cu B.Cu) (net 1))
 (via (at 114 71) (size 0.8) (drill 0.4) (layers F.Cu B.Cu) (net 1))
 (via (at 112 71) (size 0.8) (drill 0.4) (layers F.Cu B.Cu) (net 1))
 (via (at 110 71) (size 0.8) (drill 0.4) (layers F.Cu B.Cu) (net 1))
 (via (at 108 71) (size 0.8) (drill 0.4) (layers F.Cu B.Cu) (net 1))
 (via (at 101 75) (size 0.8) (drill 0.4) (layers F.Cu B.Cu) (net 1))
 (via (at 103 75) (size 0.8) (drill 0.4) (layers F.Cu B.Cu) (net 1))
 (via (at 105 75) (size 0.8) (drill 0.4) (layers F.Cu B.Cu) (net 1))
 (via (at 107 75) (size 0.8) (drill 0.4) (layers F.Cu B.Cu) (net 1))
 (via (at 109 75) (size 0.8) (drill 0.4) (layers F.Cu B.Cu) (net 1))
 (via (at 111 75) (size 0.8) (drill 0.4) (layers F.Cu B.Cu) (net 1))
 (via (at 113 75) (size 0.8) (drill 0.4) (layers F.Cu B.Cu) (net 1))
 (via (at 115 75) (size 0.8) (drill 0.4) (layers F.Cu B.Cu) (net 1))
 (via (at 117 75) (size 0.8) (drill 0.4) (layers F.Cu B.Cu) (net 1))
 (via (at 119 75) (size 0.8) (drill 0.4) (layers F.Cu B.Cu) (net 1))
 (via (at 122 75) (size 0.8) (drill 0.4) (layers F.Cu B.Cu) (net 1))
 (via (at 130 75) (size 0.8) (drill 0.4) (layers F.Cu B.Cu) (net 1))
 (via (at 132 75) (size 0.8) (drill 0.4) (layers F.Cu B.Cu) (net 1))
 (via (at 124 75) (size 0.8) (drill 0.4) (layers F.Cu B.Cu) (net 1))
 (via (at 126 75) (size 0.8) (drill 0.4) (layers F.Cu B.Cu) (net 1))
 (via (at 128 75) (size 0.8) (drill 0.4) (layers F.Cu B.Cu) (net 1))
 (via (at 106 71) (size 0.8) (drill 0.4) (layers F.Cu B.Cu) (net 1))
 (via (at 104 71) (size 0.8) (drill 0.4) (layers F.Cu B.Cu) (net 1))
 (via (at 102 71) (size 0.8) (drill 0.4) (layers F.Cu B.Cu) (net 1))
 (via (at 122 77) (size 0.8) (drill 0.4) (layers F.Cu B.Cu) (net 1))
 (via (at 123 83) (size 0.8) (drill 0.4) (layers F.Cu B.Cu) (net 1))
 (via (at 123 79) (size 0.8) (drill 0.4) (layers F.Cu B.Cu) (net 1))
 (via (at 122 85) (size 0.8) (drill 0.4) (layers F.Cu B.Cu) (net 1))
 (via (at 124 81) (size 0.8) (drill 0.4) (layers F.Cu B.Cu) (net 1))
 (via (at 110 77) (size 0.8) (drill 0.4) (layers F.Cu B.Cu) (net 1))
 (via (at 109 79) (size 0.8) (drill 0.4) (layers F.Cu B.Cu) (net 1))
 (via (at 108 81) (size 0.8) (drill 0.4) (layers F.Cu B.Cu) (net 1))
 (via (at 109 83) (size 0.8) (drill 0.4) (layers F.Cu B.Cu) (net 1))
 (via (at 110 85) (size 0.8) (drill 0.4) (layers F.Cu B.Cu) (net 1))
 (via (at 111 87) (size 0.8) (drill 0.4) (layers F.Cu B.Cu) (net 1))
 (via (at 113 87) (size 0.8) (drill 0.4) (layers F.Cu B.Cu) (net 1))
 (via (at 121 87) (size 0.8) (drill 0.4) (layers F.Cu B.Cu) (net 1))
 (via (at 124 77) (size 0.8) (drill 0.4) (layers F.Cu B.Cu) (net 1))
 (via (at 125 79) (size 0.8) (drill 0.4) (layers F.Cu B.Cu) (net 1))
 (via (at 126 81) (size 0.8) (drill 0.4) (layers F.Cu B.Cu) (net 1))
 (via (at 125 83) (size 0.8) (drill 0.4) (layers F.Cu B.Cu) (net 1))
 (via (at 124 85) (size 0.8) (drill 0.4) (layers F.Cu B.Cu) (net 1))
 (via (at 123 87) (size 0.8) (drill 0.4) (layers F.Cu B.Cu) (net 1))
 (segment (start 94.001004 69.155) (end 93.48 69.155) (width 0.25) (layer F.Cu) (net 5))
 (segment (start 94.105994 69.155) (end 97.25 72.299006) (width 0.25) (layer F.Cu) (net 5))
 (segment (start 93.48 69.155) (end 95.71499 71.38999) (width 0.75) (layer F.Cu) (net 5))
 (segment (start 96.589547 71.38999) (end 97.279778 72.080221) (width 0.75) (layer F.Cu) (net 5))
 (segment (start 95.71499 71.38999) (end 96.589547 71.38999) (width 0.75) (layer F.Cu) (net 5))
 (segment (start 98 76.2125) (end 98 74.549557) (width 0.75) (layer F.Cu) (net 5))
 (segment (start 97.300443 73.85) (end 97.25 73.85) (width 0.75) (layer F.Cu) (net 5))
 (segment (start 98 74.549557) (end 97.300443 73.85) (width 0.75) (layer F.Cu) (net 5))
 (segment (start 97.25 72.299006) (end 97.25 73.85) (width 0.25) (layer F.Cu) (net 5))
 (segment (start 85.86 69.155) (end 85.86 70.86) (width 0.25) (layer F.Cu) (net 3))
 (segment (start 85.86 70.86) (end 87.02 72.02) (width 0.25) (layer F.Cu) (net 3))
 (segment (start 87.02 76.615) (end 87 76.635) (width 0.25) (layer F.Cu) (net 3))
 (segment (start 87.02 72.02) (end 87.02 76.615) (width 0.25) (layer F.Cu) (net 3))
 (segment (start 92.614999 75.574999) (end 94.04 77) (width 0.75) (layer F.Cu) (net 3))
 (segment (start 88.060001 75.574999) (end 92.614999 75.574999) (width 0.75) (layer F.Cu) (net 3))
 (segment (start 87 76.635) (end 88.060001 75.574999) (width 0.75) (layer F.Cu) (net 3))
 (segment (start 86.429547 71.38999) (end 87.13 72.090443) (width 0.75) (layer F.Cu) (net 3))
 (segment (start 86.34499 71.38999) (end 86.429547 71.38999) (width 0.75) (layer F.Cu) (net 3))
 (segment (start 85.86 69.155) (end 85.86 70.905) (width 0.75) (layer F.Cu) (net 3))
 (segment (start 85.86 70.905) (end 86.34499 71.38999) (width 0.75) (layer F.Cu) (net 3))
 (segment (start 87 73.969557) (end 87.13 73.839557) (width 0.75) (layer F.Cu) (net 3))
 (segment (start 87 76.635) (end 87 73.969557) (width 0.75) (layer F.Cu) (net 3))
 (segment (start 91.095 76.635) (end 91.46 77) (width 0.25) (layer F.Cu) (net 4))
 (segment (start 97.362499 78.425001) (end 98 77.7875) (width 0.75) (layer F.Cu) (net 4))
 (segment (start 92.925001 78.425001) (end 97.362499 78.425001) (width 0.75) (layer F.Cu) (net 4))
 (segment (start 91.5 77) (end 92.925001 78.425001) (width 0.75) (layer F.Cu) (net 4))
 (segment (start 87 81.5) (end 91.5 77) (width 0.75) (layer F.Cu) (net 4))
 (segment (start 87 83.365) (end 87 81.5) (width 0.75) (layer F.Cu) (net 4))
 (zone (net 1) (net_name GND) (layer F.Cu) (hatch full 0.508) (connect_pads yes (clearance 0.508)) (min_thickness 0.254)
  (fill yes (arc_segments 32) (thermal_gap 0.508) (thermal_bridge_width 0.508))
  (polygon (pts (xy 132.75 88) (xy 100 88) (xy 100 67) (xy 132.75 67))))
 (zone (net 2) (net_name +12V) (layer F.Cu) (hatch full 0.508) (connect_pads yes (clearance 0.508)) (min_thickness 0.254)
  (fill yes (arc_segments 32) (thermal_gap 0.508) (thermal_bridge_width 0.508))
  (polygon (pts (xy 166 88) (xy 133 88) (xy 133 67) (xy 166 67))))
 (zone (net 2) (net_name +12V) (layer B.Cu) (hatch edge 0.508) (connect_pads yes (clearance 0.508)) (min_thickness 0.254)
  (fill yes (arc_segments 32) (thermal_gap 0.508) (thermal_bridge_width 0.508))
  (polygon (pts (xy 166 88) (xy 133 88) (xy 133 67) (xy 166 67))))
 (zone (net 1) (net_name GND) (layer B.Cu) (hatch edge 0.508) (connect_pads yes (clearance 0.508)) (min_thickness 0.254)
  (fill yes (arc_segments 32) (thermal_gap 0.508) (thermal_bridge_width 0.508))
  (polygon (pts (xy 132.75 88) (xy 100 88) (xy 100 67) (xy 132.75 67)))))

